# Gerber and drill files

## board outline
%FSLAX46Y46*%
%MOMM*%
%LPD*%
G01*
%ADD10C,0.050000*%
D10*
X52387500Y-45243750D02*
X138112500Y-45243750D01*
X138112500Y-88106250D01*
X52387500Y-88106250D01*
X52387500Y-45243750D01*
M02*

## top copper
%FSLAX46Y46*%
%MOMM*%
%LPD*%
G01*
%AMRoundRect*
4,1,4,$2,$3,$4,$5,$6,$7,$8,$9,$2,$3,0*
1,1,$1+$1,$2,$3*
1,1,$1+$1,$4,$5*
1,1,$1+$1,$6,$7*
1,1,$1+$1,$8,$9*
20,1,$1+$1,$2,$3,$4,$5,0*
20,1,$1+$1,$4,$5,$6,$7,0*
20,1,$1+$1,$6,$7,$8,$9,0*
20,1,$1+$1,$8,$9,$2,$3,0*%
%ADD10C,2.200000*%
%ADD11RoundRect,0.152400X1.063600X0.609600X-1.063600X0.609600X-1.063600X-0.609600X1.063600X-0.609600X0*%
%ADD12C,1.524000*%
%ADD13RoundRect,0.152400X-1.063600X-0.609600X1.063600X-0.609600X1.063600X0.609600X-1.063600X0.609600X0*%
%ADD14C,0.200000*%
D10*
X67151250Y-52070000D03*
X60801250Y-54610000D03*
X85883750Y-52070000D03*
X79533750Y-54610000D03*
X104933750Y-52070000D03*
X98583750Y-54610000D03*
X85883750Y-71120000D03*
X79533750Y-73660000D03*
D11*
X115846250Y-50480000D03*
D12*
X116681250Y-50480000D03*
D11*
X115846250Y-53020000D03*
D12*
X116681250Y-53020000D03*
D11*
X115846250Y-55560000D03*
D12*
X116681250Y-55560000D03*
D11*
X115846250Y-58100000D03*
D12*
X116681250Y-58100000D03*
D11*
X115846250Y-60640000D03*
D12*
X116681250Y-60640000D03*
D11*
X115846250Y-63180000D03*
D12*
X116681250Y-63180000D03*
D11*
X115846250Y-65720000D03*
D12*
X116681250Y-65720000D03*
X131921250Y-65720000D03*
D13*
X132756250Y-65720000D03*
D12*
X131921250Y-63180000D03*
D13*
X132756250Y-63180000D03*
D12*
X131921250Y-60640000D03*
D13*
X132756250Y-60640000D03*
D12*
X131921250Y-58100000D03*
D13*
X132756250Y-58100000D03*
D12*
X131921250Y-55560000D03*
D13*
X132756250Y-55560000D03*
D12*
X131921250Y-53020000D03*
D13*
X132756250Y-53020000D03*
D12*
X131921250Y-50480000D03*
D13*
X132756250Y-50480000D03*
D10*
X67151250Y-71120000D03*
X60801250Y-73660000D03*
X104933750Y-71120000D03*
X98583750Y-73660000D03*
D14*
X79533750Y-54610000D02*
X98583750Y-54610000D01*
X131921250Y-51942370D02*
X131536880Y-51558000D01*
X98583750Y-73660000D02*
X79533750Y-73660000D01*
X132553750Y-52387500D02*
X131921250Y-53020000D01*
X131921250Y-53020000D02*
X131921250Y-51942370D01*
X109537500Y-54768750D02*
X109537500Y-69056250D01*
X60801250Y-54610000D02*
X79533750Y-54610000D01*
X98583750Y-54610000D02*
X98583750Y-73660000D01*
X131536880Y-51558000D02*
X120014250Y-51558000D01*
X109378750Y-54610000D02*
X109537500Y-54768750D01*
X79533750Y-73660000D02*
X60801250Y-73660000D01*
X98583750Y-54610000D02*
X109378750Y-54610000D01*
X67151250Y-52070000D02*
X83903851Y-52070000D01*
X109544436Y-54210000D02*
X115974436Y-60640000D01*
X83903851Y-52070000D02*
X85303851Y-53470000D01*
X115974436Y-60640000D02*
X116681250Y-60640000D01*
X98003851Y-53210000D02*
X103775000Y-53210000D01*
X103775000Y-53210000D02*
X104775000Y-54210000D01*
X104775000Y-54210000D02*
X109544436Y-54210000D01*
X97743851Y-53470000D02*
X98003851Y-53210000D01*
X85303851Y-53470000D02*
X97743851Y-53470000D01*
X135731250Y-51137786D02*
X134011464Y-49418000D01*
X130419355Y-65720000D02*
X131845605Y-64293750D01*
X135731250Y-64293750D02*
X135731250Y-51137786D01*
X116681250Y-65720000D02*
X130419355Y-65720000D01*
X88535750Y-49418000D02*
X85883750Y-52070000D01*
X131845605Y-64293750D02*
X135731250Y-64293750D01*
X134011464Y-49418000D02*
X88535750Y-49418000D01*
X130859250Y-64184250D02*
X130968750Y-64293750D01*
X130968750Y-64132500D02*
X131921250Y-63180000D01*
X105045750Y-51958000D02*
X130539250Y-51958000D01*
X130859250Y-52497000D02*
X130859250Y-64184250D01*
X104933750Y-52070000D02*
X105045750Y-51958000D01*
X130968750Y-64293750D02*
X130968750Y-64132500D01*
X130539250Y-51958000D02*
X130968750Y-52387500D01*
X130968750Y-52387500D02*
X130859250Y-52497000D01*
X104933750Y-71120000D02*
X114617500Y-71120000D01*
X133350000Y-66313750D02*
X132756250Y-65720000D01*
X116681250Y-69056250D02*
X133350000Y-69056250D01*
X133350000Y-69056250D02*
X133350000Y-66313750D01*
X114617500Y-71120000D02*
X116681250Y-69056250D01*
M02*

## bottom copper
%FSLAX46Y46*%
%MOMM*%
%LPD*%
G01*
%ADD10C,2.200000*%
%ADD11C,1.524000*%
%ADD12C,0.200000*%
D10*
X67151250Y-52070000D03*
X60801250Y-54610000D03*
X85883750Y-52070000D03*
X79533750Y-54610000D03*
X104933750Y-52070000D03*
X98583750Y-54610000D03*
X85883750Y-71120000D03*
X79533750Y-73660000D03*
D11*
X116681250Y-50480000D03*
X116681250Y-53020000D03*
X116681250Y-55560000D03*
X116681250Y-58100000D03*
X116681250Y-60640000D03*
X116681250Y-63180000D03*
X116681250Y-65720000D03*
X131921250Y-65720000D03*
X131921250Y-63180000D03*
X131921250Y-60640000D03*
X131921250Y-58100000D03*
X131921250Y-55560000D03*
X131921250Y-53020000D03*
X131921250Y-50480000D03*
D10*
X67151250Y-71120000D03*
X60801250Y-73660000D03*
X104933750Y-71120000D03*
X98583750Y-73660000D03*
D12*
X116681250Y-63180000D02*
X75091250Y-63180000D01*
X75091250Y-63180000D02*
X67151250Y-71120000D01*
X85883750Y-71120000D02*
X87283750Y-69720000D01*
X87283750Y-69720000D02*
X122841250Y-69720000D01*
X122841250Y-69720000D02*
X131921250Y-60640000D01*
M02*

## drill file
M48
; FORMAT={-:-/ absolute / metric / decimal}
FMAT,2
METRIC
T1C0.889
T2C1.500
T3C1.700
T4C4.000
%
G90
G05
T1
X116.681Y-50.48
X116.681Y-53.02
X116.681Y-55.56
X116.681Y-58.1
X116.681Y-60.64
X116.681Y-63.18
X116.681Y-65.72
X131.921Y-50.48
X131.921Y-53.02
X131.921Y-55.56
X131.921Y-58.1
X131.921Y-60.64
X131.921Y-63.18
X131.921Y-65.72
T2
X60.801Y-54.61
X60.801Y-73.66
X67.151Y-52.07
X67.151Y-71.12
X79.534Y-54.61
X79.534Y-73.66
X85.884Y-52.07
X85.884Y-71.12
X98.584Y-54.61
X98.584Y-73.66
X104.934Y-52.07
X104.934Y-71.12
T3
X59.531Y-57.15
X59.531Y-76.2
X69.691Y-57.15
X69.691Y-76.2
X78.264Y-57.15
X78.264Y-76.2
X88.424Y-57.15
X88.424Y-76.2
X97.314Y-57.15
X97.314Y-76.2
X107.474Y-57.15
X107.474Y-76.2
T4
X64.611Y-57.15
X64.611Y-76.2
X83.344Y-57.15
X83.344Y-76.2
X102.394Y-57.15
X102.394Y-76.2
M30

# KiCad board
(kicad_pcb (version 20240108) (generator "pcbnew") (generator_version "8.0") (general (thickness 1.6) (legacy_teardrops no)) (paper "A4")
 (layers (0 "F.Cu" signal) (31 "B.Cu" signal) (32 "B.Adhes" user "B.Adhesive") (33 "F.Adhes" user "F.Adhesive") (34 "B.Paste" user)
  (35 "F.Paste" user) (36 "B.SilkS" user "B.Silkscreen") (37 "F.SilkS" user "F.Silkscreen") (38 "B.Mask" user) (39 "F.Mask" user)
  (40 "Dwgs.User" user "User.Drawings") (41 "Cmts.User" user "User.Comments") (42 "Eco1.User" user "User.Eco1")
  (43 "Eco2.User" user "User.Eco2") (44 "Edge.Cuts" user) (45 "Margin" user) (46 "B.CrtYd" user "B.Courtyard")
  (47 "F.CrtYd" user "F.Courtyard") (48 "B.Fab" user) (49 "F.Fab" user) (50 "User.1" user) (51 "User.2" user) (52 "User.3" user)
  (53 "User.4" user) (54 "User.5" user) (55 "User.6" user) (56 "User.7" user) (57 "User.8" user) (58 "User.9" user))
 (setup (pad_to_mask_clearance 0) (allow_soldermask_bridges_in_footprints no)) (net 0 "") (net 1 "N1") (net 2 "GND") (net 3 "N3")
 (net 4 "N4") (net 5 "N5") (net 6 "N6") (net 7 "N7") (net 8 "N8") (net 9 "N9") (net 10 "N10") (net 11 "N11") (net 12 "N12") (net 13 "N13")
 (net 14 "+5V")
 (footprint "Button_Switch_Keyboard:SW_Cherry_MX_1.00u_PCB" (layer "F.Cu") (at 67.15125 52.07)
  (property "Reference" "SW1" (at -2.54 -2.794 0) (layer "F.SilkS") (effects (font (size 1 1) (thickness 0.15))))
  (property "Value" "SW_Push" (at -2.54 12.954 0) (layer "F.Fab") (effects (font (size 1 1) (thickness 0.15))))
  (pad "" np_thru_hole circle (at -7.62 5.08) (size 1.7 1.7) (drill 1.7) (layers "*.Cu" "*.Mask"))
  (pad "" np_thru_hole circle (at -2.54 5.08) (size 4 4) (drill 4) (layers "*.Cu" "*.Mask"))
  (pad "" np_thru_hole circle (at 2.54 5.08) (size 1.7 1.7) (drill 1.7) (layers "*.Cu" "*.Mask"))
  (pad "1" thru_hole circle (at 0 0) (size 2.2 2.2) (drill 1.5) (layers "*.Cu" "*.Mask") (remove_unused_layers no) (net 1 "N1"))
  (pad "2" thru_hole circle (at -6.35 2.54) (size 2.2 2.2) (drill 1.5) (layers "*.Cu" "*.Mask") (remove_unused_layers no) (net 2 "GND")))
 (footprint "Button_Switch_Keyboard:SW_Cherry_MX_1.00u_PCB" (layer "F.Cu") (at 85.88375 52.07)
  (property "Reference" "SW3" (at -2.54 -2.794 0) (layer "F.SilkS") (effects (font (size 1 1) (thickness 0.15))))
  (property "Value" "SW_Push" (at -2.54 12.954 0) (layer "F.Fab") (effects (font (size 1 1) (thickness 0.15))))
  (pad "" np_thru_hole circle (at -7.62 5.08) (size 1.7 1.7) (drill 1.7) (layers "*.Cu" "*.Mask"))
  (pad "" np_thru_hole circle (at -2.54 5.08) (size 4 4) (drill 4) (layers "*.Cu" "*.Mask"))
  (pad "" np_thru_hole circle (at 2.54 5.08) (size 1.7 1.7) (drill 1.7) (layers "*.Cu" "*.Mask"))
  (pad "1" thru_hole circle (at 0 0) (size 2.2 2.2) (drill 1.5) (layers "*.Cu" "*.Mask") (remove_unused_layers no) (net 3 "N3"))
  (pad "2" thru_hole circle (at -6.35 2.54) (size 2.2 2.2) (drill 1.5) (layers "*.Cu" "*.Mask") (remove_unused_layers no) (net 2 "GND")))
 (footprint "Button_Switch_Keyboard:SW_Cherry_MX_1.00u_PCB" (layer "F.Cu") (at 104.93375 52.07)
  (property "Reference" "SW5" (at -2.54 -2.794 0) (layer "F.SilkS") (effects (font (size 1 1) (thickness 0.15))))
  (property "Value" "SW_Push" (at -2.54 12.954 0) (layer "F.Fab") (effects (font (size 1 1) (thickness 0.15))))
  (pad "" np_thru_hole circle (at -7.62 5.08) (size 1.7 1.7) (drill 1.7) (layers "*.Cu" "*.Mask"))
  (pad "" np_thru_hole circle (at -2.54 5.08) (size 4 4) (drill 4) (layers "*.Cu" "*.Mask"))
  (pad "" np_thru_hole circle (at 2.54 5.08) (size 1.7 1.7) (drill 1.7) (layers "*.Cu" "*.Mask"))
  (pad "1" thru_hole circle (at 0 0) (size 2.2 2.2) (drill 1.5) (layers "*.Cu" "*.Mask") (remove_unused_layers no) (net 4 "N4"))
  (pad "2" thru_hole circle (at -6.35 2.54) (size 2.2 2.2) (drill 1.5) (layers "*.Cu" "*.Mask") (remove_unused_layers no) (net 2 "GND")))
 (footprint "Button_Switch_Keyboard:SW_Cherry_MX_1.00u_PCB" (layer "F.Cu") (at 85.88375 71.12)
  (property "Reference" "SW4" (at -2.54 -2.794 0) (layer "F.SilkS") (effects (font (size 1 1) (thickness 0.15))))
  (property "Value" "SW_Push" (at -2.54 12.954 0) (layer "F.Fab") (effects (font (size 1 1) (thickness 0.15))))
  (pad "" np_thru_hole circle (at -7.62 5.08) (size 1.7 1.7) (drill 1.7) (layers "*.Cu" "*.Mask"))
  (pad "" np_thru_hole circle (at -2.54 5.08) (size 4 4) (drill 4) (layers "*.Cu" "*.Mask"))
  (pad "" np_thru_hole circle (at 2.54 5.08) (size 1.7 1.7) (drill 1.7) (layers "*.Cu" "*.Mask"))
  (pad "1" thru_hole circle (at 0 0) (size 2.2 2.2) (drill 1.5) (layers "*.Cu" "*.Mask") (remove_unused_layers no) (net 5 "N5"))
  (pad "2" thru_hole circle (at -6.35 2.54) (size 2.2 2.2) (drill 1.5) (layers "*.Cu" "*.Mask") (remove_unused_layers no) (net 2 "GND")))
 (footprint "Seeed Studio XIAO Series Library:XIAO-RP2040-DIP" (layer "F.Cu") (at 124.30125 58.1)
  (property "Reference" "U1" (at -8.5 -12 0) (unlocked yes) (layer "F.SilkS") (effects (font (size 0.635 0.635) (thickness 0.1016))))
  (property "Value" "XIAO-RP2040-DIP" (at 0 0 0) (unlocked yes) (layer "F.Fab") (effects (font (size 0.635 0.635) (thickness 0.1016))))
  (pad "1" smd roundrect (at -8.455 -7.62 180) (size 2.432 1.524) (layers "F.Cu" "F.Mask") (roundrect_rratio 0.1) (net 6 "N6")
   (thermal_bridge_angle 45))
  (pad "1" thru_hole circle (at -7.62 -7.62 180) (size 1.524 1.524) (drill 0.889) (layers "*.Cu" "*.Mask") (remove_unused_layers no)
   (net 6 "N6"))
  (pad "2" smd roundrect (at -8.455 -5.08 180) (size 2.432 1.524) (layers "F.Cu" "F.Mask") (roundrect_rratio 0.1) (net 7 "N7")
   (thermal_bridge_angle 45))
  (pad "2" thru_hole circle (at -7.62 -5.08 180) (size 1.524 1.524) (drill 0.889) (layers "*.Cu" "*.Mask") (remove_unused_layers no)
   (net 7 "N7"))
  (pad "3" smd roundrect (at -8.455 -2.54 180) (size 2.432 1.524) (layers "F.Cu" "F.Mask") (roundrect_rratio 0.1) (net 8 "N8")
   (thermal_bridge_angle 45))
  (pad "3" thru_hole circle (at -7.62 -2.54 180) (size 1.524 1.524) (drill 0.889) (layers "*.Cu" "*.Mask") (remove_unused_layers no)
   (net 8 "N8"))
  (pad "4" smd roundrect (at -8.455 0 180) (size 2.432 1.524) (layers "F.Cu" "F.Mask") (roundrect_rratio 0.1) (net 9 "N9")
   (thermal_bridge_angle 45))
  (pad "4" thru_hole circle (at -7.62 0 180) (size 1.524 1.524) (drill 0.889) (layers "*.Cu" "*.Mask") (remove_unused_layers no)
   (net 9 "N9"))
  (pad "5" smd roundrect (at -8.455 2.54 180) (size 2.432 1.524) (layers "F.Cu" "F.Mask") (roundrect_rratio 0.1) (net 1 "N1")
   (thermal_bridge_angle 45))
  (pad "5" thru_hole circle (at -7.62 2.54 180) (size 1.524 1.524) (drill 0.889) (layers "*.Cu" "*.Mask") (remove_unused_layers no)
   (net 1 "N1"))
  (pad "6" smd roundrect (at -8.455 5.08 180) (size 2.432 1.524) (layers "F.Cu" "F.Mask") (roundrect_rratio 0.1) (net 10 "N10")
   (thermal_bridge_angle 45))
  (pad "6" thru_hole circle (at -7.62 5.08 180) (size 1.524 1.524) (drill 0.889) (layers "*.Cu" "*.Mask") (remove_unused_layers no)
   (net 10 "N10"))
  (pad "7" smd roundrect (at -8.455 7.62 180) (size 2.432 1.524) (layers "F.Cu" "F.Mask") (roundrect_rratio 0.1) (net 3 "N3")
   (thermal_bridge_angle 45))
  (pad "7" thru_hole circle (at -7.62 7.62 180) (size 1.524 1.524) (drill 0.889) (layers "*.Cu" "*.Mask") (remove_unused_layers no)
   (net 3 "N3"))
  (pad "8" thru_hole circle (at 7.62 7.62) (size 1.524 1.524) (drill 0.889) (layers "*.Cu" "*.Mask") (remove_unused_layers no)
   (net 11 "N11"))
  (pad "8" smd roundrect (at 8.455 7.62) (size 2.432 1.524) (layers "F.Cu" "F.Mask") (roundrect_rratio 0.1) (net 11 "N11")
   (thermal_bridge_angle 45))
  (pad "9" thru_hole circle (at 7.62 5.08) (size 1.524 1.524) (drill 0.889) (layers "*.Cu" "*.Mask") (remove_unused_layers no) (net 4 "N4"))
  (pad "9" smd roundrect (at 8.455 5.08) (size 2.432 1.524) (layers "F.Cu" "F.Mask") (roundrect_rratio 0.1) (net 4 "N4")
   (thermal_bridge_angle 45))
  (pad "10" thru_hole circle (at 7.62 2.54) (size 1.524 1.524) (drill 0.889) (layers "*.Cu" "*.Mask") (remove_unused_layers no) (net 5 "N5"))
  (pad "10" smd roundrect (at 8.455 2.54) (size 2.432 1.524) (layers "F.Cu" "F.Mask") (roundrect_rratio 0.1) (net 5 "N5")
   (thermal_bridge_angle 45))
  (pad "11" thru_hole circle (at 7.62 0) (size 1.524 1.524) (drill 0.889) (layers "*.Cu" "*.Mask") (remove_unused_layers no) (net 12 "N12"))
  (pad "11" smd roundrect (at 8.455 0) (size 2.432 1.524) (layers "F.Cu" "F.Mask") (roundrect_rratio 0.1) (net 12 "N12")
   (thermal_bridge_angle 45))
  (pad "12" thru_hole circle (at 7.62 -2.54) (size 1.524 1.524) (drill 0.889) (layers "*.Cu" "*.Mask") (remove_unused_layers no)
   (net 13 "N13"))
  (pad "12" smd roundrect (at 8.455 -2.54) (size 2.432 1.524) (layers "F.Cu" "F.Mask") (roundrect_rratio 0.1) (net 13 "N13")
   (thermal_bridge_angle 45))
  (pad "13" thru_hole circle (at 7.62 -5.08) (size 1.524 1.524) (drill 0.889) (layers "*.Cu" "*.Mask") (remove_unused_layers no)
   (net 2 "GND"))
  (pad "13" smd roundrect (at 8.455 -5.08) (size 2.432 1.524) (layers "F.Cu" "F.Mask") (roundrect_rratio 0.1) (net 2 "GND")
   (thermal_bridge_angle 45))
  (pad "14" thru_hole circle (at 7.62 -7.62) (size 1.524 1.524) (drill 0.889) (layers "*.Cu" "*.Mask") (remove_unused_layers no)
   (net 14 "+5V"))
  (pad "14" smd roundrect (at 8.455 -7.62) (size 2.432 1.524) (layers "F.Cu" "F.Mask") (roundrect_rratio 0.1) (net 14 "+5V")
   (thermal_bridge_angle 45)))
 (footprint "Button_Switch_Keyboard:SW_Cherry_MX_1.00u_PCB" (layer "F.Cu") (at 67.15125 71.12)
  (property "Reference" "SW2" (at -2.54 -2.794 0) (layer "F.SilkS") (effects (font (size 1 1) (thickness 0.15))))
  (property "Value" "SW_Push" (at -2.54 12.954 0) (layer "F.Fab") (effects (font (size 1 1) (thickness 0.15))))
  (pad "" np_thru_hole circle (at -7.62 5.08) (size 1.7 1.7) (drill 1.7) (layers "*.Cu" "*.Mask"))
  (pad "" np_thru_hole circle (at -2.54 5.08) (size 4 4) (drill 4) (layers "*.Cu" "*.Mask"))
  (pad "" np_thru_hole circle (at 2.54 5.08) (size 1.7 1.7) (drill 1.7) (layers "*.Cu" "*.Mask"))
  (pad "1" thru_hole circle (at 0 0) (size 2.2 2.2) (drill 1.5) (layers "*.Cu" "*.Mask") (remove_unused_layers no) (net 10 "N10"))
  (pad "2" thru_hole circle (at -6.35 2.54) (size 2.2 2.2) (drill 1.5) (layers "*.Cu" "*.Mask") (remove_unused_layers no) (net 2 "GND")))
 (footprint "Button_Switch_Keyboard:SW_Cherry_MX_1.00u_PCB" (layer "F.Cu") (at 104.93375 71.12)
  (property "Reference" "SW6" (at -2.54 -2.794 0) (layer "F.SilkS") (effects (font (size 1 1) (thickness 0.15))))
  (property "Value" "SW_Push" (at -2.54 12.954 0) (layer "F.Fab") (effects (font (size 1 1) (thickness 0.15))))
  (pad "" np_thru_hole circle (at -7.62 5.08) (size 1.7 1.7) (drill 1.7) (layers "*.Cu" "*.Mask"))
  (pad "" np_thru_hole circle (at -2.54 5.08) (size 4 4) (drill 4) (layers "*.Cu" "*.Mask"))
  (pad "" np_thru_hole circle (at 2.54 5.08) (size 1.7 1.7) (drill 1.7) (layers "*.Cu" "*.Mask"))
  (pad "1" thru_hole circle (at 0 0) (size 2.2 2.2) (drill 1.5) (layers "*.Cu" "*.Mask") (remove_unused_layers no) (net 11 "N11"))
  (pad "2" thru_hole circle (at -6.35 2.54) (size 2.2 2.2) (drill 1.5) (layers "*.Cu" "*.Mask") (remove_unused_layers no) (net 2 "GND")))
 (gr_rect (start 52.3875 45.24375) (end 138.1125 88.10625) (stroke (width 0.05) (type default)) (fill none) (layer "Edge.Cuts"))
 (segment (start 79.53375 54.61) (end 98.58375 54.61) (width 0.2) (layer "F.Cu") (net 2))
 (segment (start 131.92125 51.94237) (end 131.53688 51.558) (width 0.2) (layer "F.Cu") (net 2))
 (segment (start 98.58375 73.66) (end 79.53375 73.66) (width 0.2) (layer "F.Cu") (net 2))
 (segment (start 132.55375 52.3875) (end 131.92125 53.02) (width 0.2) (layer "F.Cu") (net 2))
 (segment (start 131.92125 53.02) (end 131.92125 51.94237) (width 0.2) (layer "F.Cu") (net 2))
 (segment (start 109.5375 54.76875) (end 109.5375 69.05625) (width 0.2) (layer "F.Cu") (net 2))
 (segment (start 60.80125 54.61) (end 79.53375 54.61) (width 0.2) (layer "F.Cu") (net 2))
 (segment (start 98.58375 54.61) (end 98.58375 73.66) (width 0.2) (layer "F.Cu") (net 2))
 (segment (start 131.53688 51.558) (end 120.01425 51.558) (width 0.2) (layer "F.Cu") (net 2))
 (segment (start 109.37875 54.61) (end 109.5375 54.76875) (width 0.2) (layer "F.Cu") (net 2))
 (segment (start 79.53375 73.66) (end 60.80125 73.66) (width 0.2) (layer "F.Cu") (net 2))
 (segment (start 98.58375 54.61) (end 109.37875 54.61) (width 0.2) (layer "F.Cu") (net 2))
 (segment (start 67.15125 52.07) (end 83.903851 52.07) (width 0.2) (layer "F.Cu") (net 1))
 (segment (start 109.544436 54.21) (end 115.974436 60.64) (width 0.2) (layer "F.Cu") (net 1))
 (segment (start 83.903851 52.07) (end 85.303851 53.47) (width 0.2) (layer "F.Cu") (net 1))
 (segment (start 115.974436 60.64) (end 116.68125 60.64) (width 0.2) (layer "F.Cu") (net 1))
 (segment (start 98.003851 53.21) (end 103.775 53.21) (width 0.2) (layer "F.Cu") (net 1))
 (segment (start 103.775 53.21) (end 104.775 54.21) (width 0.2) (layer "F.Cu") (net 1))
 (segment (start 104.775 54.21) (end 109.544436 54.21) (width 0.2) (layer "F.Cu") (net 1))
 (segment (start 97.743851 53.47) (end 98.003851 53.21) (width 0.2) (layer "F.Cu") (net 1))
 (segment (start 85.303851 53.47) (end 97.743851 53.47) (width 0.2) (layer "F.Cu") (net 1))
 (segment (start 116.68125 63.18) (end 75.09125 63.18) (width 0.2) (layer "B.Cu") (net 10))
 (segment (start 75.09125 63.18) (end 67.15125 71.12) (width 0.2) (layer "B.Cu") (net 10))
 (segment (start 135.73125 51.137786) (end 134.011464 49.418) (width 0.2) (layer "F.Cu") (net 3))
 (segment (start 130.419355 65.72) (end 131.845605 64.29375) (width 0.2) (layer "F.Cu") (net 3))
 (segment (start 135.73125 64.29375) (end 135.73125 51.137786) (width 0.2) (layer "F.Cu") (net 3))
 (segment (start 116.68125 65.72) (end 130.419355 65.72) (width 0.2) (layer "F.Cu") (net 3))
 (segment (start 88.53575 49.418) (end 85.88375 52.07) (width 0.2) (layer "F.Cu") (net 3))
 (segment (start 131.845605 64.29375) (end 135.73125 64.29375) (width 0.2) (layer "F.Cu") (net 3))
 (segment (start 134.011464 49.418) (end 88.53575 49.418) (width 0.2) (layer "F.Cu") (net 3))
 (segment (start 85.88375 71.12) (end 87.28375 69.72) (width 0.2) (layer "B.Cu") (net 5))
 (segment (start 87.28375 69.72) (end 122.84125 69.72) (width 0.2) (layer "B.Cu") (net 5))
 (segment (start 122.84125 69.72) (end 131.92125 60.64) (width 0.2) (layer "B.Cu") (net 5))
 (segment (start 130.85925 64.18425) (end 130.96875 64.29375) (width 0.2) (layer "F.Cu") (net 4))
 (segment (start 130.96875 64.1325) (end 131.92125 63.18) (width 0.2) (layer "F.Cu") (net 4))
 (segment (start 105.04575 51.958) (end 130.53925 51.958) (width 0.2) (layer "F.Cu") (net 4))
 (segment (start 130.85925 52.497) (end 130.85925 64.18425) (width 0.2) (layer "F.Cu") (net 4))
 (segment (start 104.93375 52.07) (end 105.04575 51.958) (width 0.2) (layer "F.Cu") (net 4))
 (segment (start 130.96875 64.29375) (end 130.96875 64.1325) (width 0.2) (layer "F.Cu") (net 4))
 (segment (start 130.53925 51.958) (end 130.96875 52.3875) (width 0.2) (layer "F.Cu") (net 4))
 (segment (start 130.96875 52.3875) (end 130.85925 52.497) (width 0.2) (layer "F.Cu") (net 4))
 (segment (start 104.93375 71.12) (end 114.6175 71.12) (width 0.2) (layer "F.Cu") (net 11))
 (segment (start 133.35 66.31375) (end 132.75625 65.72) (width 0.2) (layer "F.Cu") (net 11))
 (segment (start 116.68125 69.05625) (end 133.35 69.05625) (width 0.2) (layer "F.Cu") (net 11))
 (segment (start 133.35 69.05625) (end 133.35 66.31375) (width 0.2) (layer "F.Cu") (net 11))
 (segment (start 114.6175 71.12) (end 116.68125 69.05625) (width 0.2) (layer "F.Cu") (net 11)))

